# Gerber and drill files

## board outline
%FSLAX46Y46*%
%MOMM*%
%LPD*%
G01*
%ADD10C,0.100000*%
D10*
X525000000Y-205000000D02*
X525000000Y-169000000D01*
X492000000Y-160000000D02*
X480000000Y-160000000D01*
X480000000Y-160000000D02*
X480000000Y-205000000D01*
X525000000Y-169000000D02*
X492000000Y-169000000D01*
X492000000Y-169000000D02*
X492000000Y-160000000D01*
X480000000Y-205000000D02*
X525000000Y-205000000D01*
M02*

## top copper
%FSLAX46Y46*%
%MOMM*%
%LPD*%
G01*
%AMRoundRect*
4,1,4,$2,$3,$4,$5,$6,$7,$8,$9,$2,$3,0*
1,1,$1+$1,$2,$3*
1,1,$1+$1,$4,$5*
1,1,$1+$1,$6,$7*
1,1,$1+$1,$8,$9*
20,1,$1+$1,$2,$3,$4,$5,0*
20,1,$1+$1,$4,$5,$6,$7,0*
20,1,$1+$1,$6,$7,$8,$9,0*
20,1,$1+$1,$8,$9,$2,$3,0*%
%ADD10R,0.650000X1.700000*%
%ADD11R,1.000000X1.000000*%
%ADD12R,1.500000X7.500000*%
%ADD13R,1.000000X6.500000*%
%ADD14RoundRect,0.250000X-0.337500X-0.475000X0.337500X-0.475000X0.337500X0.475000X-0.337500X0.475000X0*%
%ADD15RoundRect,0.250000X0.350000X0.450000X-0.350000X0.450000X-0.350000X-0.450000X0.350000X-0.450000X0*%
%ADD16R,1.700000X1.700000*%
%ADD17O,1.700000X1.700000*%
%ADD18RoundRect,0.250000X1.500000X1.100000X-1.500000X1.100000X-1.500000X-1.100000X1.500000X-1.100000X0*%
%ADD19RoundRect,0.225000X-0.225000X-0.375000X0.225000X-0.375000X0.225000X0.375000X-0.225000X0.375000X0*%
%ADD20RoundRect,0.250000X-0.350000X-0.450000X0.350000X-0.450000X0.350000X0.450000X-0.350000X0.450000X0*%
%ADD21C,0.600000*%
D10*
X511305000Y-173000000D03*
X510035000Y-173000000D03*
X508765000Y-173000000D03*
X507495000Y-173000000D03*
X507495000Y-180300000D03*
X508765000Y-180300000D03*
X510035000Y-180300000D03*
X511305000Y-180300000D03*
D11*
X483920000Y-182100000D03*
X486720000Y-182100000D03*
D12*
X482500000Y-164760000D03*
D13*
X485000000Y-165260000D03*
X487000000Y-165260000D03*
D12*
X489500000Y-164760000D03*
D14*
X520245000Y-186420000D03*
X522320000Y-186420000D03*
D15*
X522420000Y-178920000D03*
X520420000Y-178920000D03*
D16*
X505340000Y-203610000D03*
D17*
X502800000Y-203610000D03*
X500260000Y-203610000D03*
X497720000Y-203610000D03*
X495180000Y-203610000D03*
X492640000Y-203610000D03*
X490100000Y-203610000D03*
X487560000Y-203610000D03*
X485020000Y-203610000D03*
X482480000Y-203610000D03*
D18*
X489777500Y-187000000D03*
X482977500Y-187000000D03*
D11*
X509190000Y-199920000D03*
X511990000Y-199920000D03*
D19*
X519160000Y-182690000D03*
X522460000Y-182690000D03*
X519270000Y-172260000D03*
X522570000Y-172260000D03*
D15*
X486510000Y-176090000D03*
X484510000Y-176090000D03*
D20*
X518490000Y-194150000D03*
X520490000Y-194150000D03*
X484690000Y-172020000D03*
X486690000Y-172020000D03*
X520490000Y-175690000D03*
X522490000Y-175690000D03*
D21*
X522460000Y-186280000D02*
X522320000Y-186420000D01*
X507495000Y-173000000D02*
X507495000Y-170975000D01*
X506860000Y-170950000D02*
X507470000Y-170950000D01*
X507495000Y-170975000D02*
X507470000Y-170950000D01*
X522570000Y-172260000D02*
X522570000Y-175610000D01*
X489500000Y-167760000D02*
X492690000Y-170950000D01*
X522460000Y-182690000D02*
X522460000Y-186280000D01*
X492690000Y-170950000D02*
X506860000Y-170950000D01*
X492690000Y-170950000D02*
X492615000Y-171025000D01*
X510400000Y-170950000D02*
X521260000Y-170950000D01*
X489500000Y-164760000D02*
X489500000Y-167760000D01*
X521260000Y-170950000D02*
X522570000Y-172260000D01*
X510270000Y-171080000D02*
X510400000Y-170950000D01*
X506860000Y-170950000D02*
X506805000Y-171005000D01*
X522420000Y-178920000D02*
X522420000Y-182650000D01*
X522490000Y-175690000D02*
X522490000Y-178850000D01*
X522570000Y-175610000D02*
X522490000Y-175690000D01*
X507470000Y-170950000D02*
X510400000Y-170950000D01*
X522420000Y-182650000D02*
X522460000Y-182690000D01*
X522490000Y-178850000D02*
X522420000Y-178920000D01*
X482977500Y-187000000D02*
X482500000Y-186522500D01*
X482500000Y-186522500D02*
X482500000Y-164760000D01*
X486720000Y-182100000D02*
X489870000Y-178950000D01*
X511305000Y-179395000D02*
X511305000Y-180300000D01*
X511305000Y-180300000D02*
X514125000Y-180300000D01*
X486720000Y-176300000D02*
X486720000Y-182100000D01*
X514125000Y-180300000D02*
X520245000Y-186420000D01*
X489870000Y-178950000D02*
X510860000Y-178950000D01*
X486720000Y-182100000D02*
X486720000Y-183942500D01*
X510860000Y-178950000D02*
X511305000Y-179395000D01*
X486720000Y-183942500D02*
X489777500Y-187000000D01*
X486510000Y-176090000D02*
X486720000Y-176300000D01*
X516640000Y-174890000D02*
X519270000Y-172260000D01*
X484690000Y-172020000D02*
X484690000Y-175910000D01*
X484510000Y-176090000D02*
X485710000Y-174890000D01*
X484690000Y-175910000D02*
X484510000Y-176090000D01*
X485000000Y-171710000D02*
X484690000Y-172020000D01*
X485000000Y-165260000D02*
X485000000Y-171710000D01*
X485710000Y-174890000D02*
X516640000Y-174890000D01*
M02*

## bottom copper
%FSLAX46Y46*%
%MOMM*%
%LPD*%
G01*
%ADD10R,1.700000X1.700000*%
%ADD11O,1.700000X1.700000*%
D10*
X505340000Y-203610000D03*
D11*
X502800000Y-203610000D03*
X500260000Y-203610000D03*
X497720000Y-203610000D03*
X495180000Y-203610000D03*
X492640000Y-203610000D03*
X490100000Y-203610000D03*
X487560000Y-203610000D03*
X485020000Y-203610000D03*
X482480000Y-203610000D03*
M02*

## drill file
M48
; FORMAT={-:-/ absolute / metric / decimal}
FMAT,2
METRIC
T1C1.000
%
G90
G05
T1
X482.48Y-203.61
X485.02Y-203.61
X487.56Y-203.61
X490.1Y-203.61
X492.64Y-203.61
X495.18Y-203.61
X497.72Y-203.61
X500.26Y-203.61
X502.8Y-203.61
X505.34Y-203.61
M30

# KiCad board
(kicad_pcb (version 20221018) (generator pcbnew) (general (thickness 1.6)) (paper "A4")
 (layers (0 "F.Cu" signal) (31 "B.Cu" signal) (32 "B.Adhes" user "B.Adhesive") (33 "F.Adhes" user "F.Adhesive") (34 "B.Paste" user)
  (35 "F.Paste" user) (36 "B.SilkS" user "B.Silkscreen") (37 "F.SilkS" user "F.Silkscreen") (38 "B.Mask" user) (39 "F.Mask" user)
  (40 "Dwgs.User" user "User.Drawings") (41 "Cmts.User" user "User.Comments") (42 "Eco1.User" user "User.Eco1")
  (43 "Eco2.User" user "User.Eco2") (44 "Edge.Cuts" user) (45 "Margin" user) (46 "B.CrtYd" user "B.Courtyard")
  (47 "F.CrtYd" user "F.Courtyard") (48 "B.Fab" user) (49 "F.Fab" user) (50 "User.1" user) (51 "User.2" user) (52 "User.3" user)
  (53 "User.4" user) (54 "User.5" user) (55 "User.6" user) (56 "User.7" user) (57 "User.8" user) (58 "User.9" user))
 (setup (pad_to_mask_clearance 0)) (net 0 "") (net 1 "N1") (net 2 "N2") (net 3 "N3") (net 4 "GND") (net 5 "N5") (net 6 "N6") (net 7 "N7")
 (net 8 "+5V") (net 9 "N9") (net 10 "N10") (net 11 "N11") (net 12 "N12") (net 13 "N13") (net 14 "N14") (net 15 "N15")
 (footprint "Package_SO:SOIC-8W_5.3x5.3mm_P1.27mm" (layer "F.Cu") (at 509.4 176.65 -90)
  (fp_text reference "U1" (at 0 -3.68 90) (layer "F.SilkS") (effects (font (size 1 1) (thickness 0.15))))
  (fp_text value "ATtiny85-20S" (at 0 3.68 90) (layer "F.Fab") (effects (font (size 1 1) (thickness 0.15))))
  (pad "1" smd rect (at -3.65 -1.905 270) (size 1.7 0.65) (layers "F.Cu" "F.Paste" "F.Mask") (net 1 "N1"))
  (pad "2" smd rect (at -3.65 -0.635 270) (size 1.7 0.65) (layers "F.Cu" "F.Paste" "F.Mask") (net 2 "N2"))
  (pad "3" smd rect (at -3.65 0.635 270) (size 1.7 0.65) (layers "F.Cu" "F.Paste" "F.Mask") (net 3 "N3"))
  (pad "4" smd rect (at -3.65 1.905 270) (size 1.7 0.65) (layers "F.Cu" "F.Paste" "F.Mask") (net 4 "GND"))
  (pad "5" smd rect (at 3.65 1.905 270) (size 1.7 0.65) (layers "F.Cu" "F.Paste" "F.Mask") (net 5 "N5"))
  (pad "6" smd rect (at 3.65 0.635 270) (size 1.7 0.65) (layers "F.Cu" "F.Paste" "F.Mask") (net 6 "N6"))
  (pad "7" smd rect (at 3.65 -0.635 270) (size 1.7 0.65) (layers "F.Cu" "F.Paste" "F.Mask") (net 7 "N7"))
  (pad "8" smd rect (at 3.65 -1.905 270) (size 1.7 0.65) (layers "F.Cu" "F.Paste" "F.Mask") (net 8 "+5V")))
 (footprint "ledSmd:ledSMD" (layer "F.Cu") (at 485.72 182.1)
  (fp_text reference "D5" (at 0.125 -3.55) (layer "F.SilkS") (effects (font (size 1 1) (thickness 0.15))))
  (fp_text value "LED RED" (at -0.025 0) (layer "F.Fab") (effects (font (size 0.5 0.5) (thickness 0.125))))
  (pad "1" smd rect (at -1.8 0) (size 1 1) (layers "F.Cu" "F.Paste" "F.Mask") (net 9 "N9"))
  (pad "2" smd rect (at 1 0) (size 1 1) (layers "F.Cu" "F.Paste" "F.Mask") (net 8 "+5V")))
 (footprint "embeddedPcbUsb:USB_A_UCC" (layer "F.Cu") (at 486 164.96 -90)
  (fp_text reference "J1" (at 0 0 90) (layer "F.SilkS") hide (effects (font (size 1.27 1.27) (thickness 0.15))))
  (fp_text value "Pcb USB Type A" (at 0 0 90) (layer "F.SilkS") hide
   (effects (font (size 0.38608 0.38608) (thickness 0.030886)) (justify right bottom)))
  (pad "1" smd rect (at -0.2 3.5 270) (size 7.5 1.5) (layers "F.Cu" "F.Paste" "F.Mask") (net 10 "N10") (solder_mask_margin 0.1016))
  (pad "2" smd rect (at 0.3 1 270) (size 6.5 1) (layers "F.Cu" "F.Paste" "F.Mask") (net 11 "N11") (solder_mask_margin 0.1016))
  (pad "3" smd rect (at 0.3 -1 270) (size 6.5 1) (layers "F.Cu" "F.Paste" "F.Mask") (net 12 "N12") (solder_mask_margin 0.1016))
  (pad "4" smd rect (at -0.2 -3.5 270) (size 7.5 1.5) (layers "F.Cu" "F.Paste" "F.Mask") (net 4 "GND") (solder_mask_margin 0.1016)))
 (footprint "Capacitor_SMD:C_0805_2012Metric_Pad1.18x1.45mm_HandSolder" (layer "F.Cu") (at 521.2825 186.42)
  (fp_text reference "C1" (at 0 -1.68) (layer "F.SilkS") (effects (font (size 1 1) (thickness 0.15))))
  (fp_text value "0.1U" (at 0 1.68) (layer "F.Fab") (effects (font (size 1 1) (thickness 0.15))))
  (pad "1" smd roundrect (at -1.0375 0) (size 1.175 1.45) (layers "F.Cu" "F.Paste" "F.Mask") (roundrect_rratio 0.212766) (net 8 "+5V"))
  (pad "2" smd roundrect (at 1.0375 0) (size 1.175 1.45) (layers "F.Cu" "F.Paste" "F.Mask") (roundrect_rratio 0.212766) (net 4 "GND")))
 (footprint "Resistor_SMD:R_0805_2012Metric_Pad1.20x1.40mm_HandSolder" (layer "F.Cu") (at 521.42 178.92 180)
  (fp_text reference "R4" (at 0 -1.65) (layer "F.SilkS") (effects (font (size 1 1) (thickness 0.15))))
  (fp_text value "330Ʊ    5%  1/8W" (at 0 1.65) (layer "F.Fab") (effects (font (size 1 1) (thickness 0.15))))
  (pad "1" smd roundrect (at -1 0 180) (size 1.2 1.4) (layers "F.Cu" "F.Paste" "F.Mask") (roundrect_rratio 0.208333) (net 4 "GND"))
  (pad "2" smd roundrect (at 1 0 180) (size 1.2 1.4) (layers "F.Cu" "F.Paste" "F.Mask") (roundrect_rratio 0.208333) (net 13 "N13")))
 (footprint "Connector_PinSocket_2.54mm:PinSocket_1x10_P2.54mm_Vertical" (layer "F.Cu") (at 505.34 203.61 -90)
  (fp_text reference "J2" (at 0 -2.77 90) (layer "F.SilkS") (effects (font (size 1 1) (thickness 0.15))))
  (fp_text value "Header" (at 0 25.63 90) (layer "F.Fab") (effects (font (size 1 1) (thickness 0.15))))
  (pad "1" thru_hole rect (at 0 0 270) (size 1.7 1.7) (drill 1) (layers "*.Cu" "*.Mask") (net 8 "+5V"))
  (pad "2" thru_hole oval (at 0 2.54 270) (size 1.7 1.7) (drill 1) (layers "*.Cu" "*.Mask") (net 4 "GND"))
  (pad "3" thru_hole oval (at 0 5.08 270) (size 1.7 1.7) (drill 1) (layers "*.Cu" "*.Mask") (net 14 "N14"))
  (pad "4" thru_hole oval (at 0 7.62 270) (size 1.7 1.7) (drill 1) (layers "*.Cu" "*.Mask") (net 5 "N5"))
  (pad "5" thru_hole oval (at 0 10.16 270) (size 1.7 1.7) (drill 1) (layers "*.Cu" "*.Mask") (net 6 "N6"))
  (pad "6" thru_hole oval (at 0 12.7 270) (size 1.7 1.7) (drill 1) (layers "*.Cu" "*.Mask") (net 7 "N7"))
  (pad "7" thru_hole oval (at 0 15.24 270) (size 1.7 1.7) (drill 1) (layers "*.Cu" "*.Mask") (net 2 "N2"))
  (pad "8" thru_hole oval (at 0 17.78 270) (size 1.7 1.7) (drill 1) (layers "*.Cu" "*.Mask") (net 3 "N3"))
  (pad "9" thru_hole oval (at 0 20.32 270) (size 1.7 1.7) (drill 1) (layers "*.Cu" "*.Mask") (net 1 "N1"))
  (pad "10" thru_hole oval (at 0 22.86 270) (size 1.7 1.7) (drill 1) (layers "*.Cu" "*.Mask") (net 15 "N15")))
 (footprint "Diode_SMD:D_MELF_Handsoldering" (layer "F.Cu") (at 486.3775 187 180)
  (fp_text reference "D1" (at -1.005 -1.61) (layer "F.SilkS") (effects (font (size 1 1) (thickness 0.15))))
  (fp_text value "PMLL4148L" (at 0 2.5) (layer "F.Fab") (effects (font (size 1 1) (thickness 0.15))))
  (pad "1" smd roundrect (at -3.4 0 180) (size 3.5 2.7) (layers "F.Cu" "F.Paste" "F.Mask") (roundrect_rratio 0.0925925926) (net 8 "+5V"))
  (pad "2" smd roundrect (at 3.4 0 180) (size 3.5 2.7) (layers "F.Cu" "F.Paste" "F.Mask") (roundrect_rratio 0.0925925926) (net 10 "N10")))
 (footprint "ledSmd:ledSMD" (layer "F.Cu") (at 510.99 199.92)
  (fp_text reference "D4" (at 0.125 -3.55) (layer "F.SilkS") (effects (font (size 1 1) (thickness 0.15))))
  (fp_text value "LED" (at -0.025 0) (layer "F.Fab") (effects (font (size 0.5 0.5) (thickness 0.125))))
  (pad "1" smd rect (at -1.8 0) (size 1 1) (layers "F.Cu" "F.Paste" "F.Mask") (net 13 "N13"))
  (pad "2" smd rect (at 1 0) (size 1 1) (layers "F.Cu" "F.Paste" "F.Mask") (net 6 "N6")))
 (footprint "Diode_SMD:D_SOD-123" (layer "F.Cu") (at 520.81 182.69)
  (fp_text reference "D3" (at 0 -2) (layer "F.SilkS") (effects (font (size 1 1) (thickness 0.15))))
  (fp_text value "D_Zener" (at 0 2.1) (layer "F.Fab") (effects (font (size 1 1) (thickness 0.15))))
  (pad "1" smd roundrect (at -1.65 0) (size 0.9 1.2) (layers "F.Cu" "F.Paste" "F.Mask") (roundrect_rratio 0.25) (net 12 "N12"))
  (pad "2" smd roundrect (at 1.65 0) (size 0.9 1.2) (layers "F.Cu" "F.Paste" "F.Mask") (roundrect_rratio 0.25) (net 4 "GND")))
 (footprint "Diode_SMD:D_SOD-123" (layer "F.Cu") (at 520.92 172.26)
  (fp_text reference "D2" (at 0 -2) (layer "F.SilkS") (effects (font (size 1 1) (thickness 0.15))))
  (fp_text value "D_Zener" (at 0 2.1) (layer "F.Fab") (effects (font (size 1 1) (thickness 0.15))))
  (pad "1" smd roundrect (at -1.65 0) (size 0.9 1.2) (layers "F.Cu" "F.Paste" "F.Mask") (roundrect_rratio 0.25) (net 11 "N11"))
  (pad "2" smd roundrect (at 1.65 0) (size 0.9 1.2) (layers "F.Cu" "F.Paste" "F.Mask") (roundrect_rratio 0.25) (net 4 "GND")))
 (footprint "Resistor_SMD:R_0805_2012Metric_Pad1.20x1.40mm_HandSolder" (layer "F.Cu") (at 485.51 176.09 180)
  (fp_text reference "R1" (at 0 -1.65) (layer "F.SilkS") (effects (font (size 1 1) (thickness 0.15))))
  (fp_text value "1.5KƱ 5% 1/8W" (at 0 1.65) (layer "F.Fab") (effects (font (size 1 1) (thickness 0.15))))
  (pad "1" smd roundrect (at -1 0 180) (size 1.2 1.4) (layers "F.Cu" "F.Paste" "F.Mask") (roundrect_rratio 0.208333) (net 8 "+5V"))
  (pad "2" smd roundrect (at 1 0 180) (size 1.2 1.4) (layers "F.Cu" "F.Paste" "F.Mask") (roundrect_rratio 0.208333) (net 11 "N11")))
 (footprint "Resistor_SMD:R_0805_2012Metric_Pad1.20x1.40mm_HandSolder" (layer "F.Cu") (at 519.49 194.15)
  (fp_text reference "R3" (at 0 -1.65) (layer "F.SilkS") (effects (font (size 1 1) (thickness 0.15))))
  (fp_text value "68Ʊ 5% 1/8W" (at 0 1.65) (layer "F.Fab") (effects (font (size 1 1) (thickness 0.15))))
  (pad "1" smd roundrect (at -1 0) (size 1.2 1.4) (layers "F.Cu" "F.Paste" "F.Mask") (roundrect_rratio 0.208333) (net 12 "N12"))
  (pad "2" smd roundrect (at 1 0) (size 1.2 1.4) (layers "F.Cu" "F.Paste" "F.Mask") (roundrect_rratio 0.208333) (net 3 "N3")))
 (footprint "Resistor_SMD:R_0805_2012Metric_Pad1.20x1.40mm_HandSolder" (layer "F.Cu") (at 485.69 172.02)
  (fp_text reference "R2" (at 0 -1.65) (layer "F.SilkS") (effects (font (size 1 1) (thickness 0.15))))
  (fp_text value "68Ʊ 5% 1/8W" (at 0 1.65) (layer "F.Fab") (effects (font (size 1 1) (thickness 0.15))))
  (pad "1" smd roundrect (at -1 0) (size 1.2 1.4) (layers "F.Cu" "F.Paste" "F.Mask") (roundrect_rratio 0.208333) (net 11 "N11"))
  (pad "2" smd roundrect (at 1 0) (size 1.2 1.4) (layers "F.Cu" "F.Paste" "F.Mask") (roundrect_rratio 0.208333) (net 2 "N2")))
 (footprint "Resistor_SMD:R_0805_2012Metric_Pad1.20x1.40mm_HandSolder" (layer "F.Cu") (at 521.49 175.69)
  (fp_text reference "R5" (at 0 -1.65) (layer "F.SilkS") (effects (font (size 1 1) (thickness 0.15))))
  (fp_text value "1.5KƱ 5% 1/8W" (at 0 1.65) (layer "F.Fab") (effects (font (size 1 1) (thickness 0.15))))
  (pad "1" smd roundrect (at -1 0) (size 1.2 1.4) (layers "F.Cu" "F.Paste" "F.Mask") (roundrect_rratio 0.208333) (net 9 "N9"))
  (pad "2" smd roundrect (at 1 0) (size 1.2 1.4) (layers "F.Cu" "F.Paste" "F.Mask") (roundrect_rratio 0.208333) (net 4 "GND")))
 (gr_line (start 525 205) (end 525 169) (stroke (width 0.1) (type default)) (layer "Edge.Cuts"))
 (gr_line (start 492 160) (end 480 160) (stroke (width 0.1) (type default)) (layer "Edge.Cuts"))
 (gr_line (start 480 160) (end 480 205) (stroke (width 0.1) (type default)) (layer "Edge.Cuts"))
 (gr_line (start 525 169) (end 492 169) (stroke (width 0.1) (type default)) (layer "Edge.Cuts"))
 (gr_line (start 492 169) (end 492 160) (stroke (width 0.1) (type default)) (layer "Edge.Cuts"))
 (gr_line (start 480 205) (end 525 205) (stroke (width 0.1) (type default)) (layer "Edge.Cuts"))
 (segment (start 522.46 186.28) (end 522.32 186.42) (width 0.6) (layer "F.Cu") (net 4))
 (segment (start 507.495 173) (end 507.495 170.975) (width 0.6) (layer "F.Cu") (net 4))
 (segment (start 506.86 170.95) (end 507.47 170.95) (width 0.6) (layer "F.Cu") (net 4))
 (segment (start 507.495 170.975) (end 507.47 170.95) (width 0.6) (layer "F.Cu") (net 4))
 (segment (start 522.57 172.26) (end 522.57 175.61) (width 0.6) (layer "F.Cu") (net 4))
 (segment (start 489.5 167.76) (end 492.69 170.95) (width 0.6) (layer "F.Cu") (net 4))
 (segment (start 522.46 182.69) (end 522.46 186.28) (width 0.6) (layer "F.Cu") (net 4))
 (segment (start 492.69 170.95) (end 506.86 170.95) (width 0.6) (layer "F.Cu") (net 4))
 (segment (start 492.69 170.95) (end 492.615 171.025) (width 0.6) (layer "F.Cu") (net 4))
 (segment (start 510.4 170.95) (end 521.26 170.95) (width 0.6) (layer "F.Cu") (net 4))
 (segment (start 489.5 164.76) (end 489.5 167.76) (width 0.6) (layer "F.Cu") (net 4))
 (segment (start 521.26 170.95) (end 522.57 172.26) (width 0.6) (layer "F.Cu") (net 4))
 (segment (start 510.27 171.08) (end 510.4 170.95) (width 0.6) (layer "F.Cu") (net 4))
 (segment (start 506.86 170.95) (end 506.805 171.005) (width 0.6) (layer "F.Cu") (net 4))
 (segment (start 522.42 178.92) (end 522.42 182.65) (width 0.6) (layer "F.Cu") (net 4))
 (segment (start 522.49 175.69) (end 522.49 178.85) (width 0.6) (layer "F.Cu") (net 4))
 (segment (start 522.57 175.61) (end 522.49 175.69) (width 0.6) (layer "F.Cu") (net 4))
 (segment (start 507.47 170.95) (end 510.4 170.95) (width 0.6) (layer "F.Cu") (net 4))
 (segment (start 522.42 182.65) (end 522.46 182.69) (width 0.6) (layer "F.Cu") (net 4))
 (segment (start 522.49 178.85) (end 522.42 178.92) (width 0.6) (layer "F.Cu") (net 4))
 (segment (start 482.9775 187) (end 482.5 186.5225) (width 0.6) (layer "F.Cu") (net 10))
 (segment (start 482.5 186.5225) (end 482.5 164.76) (width 0.6) (layer "F.Cu") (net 10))
 (segment (start 486.72 182.1) (end 489.87 178.95) (width 0.6) (layer "F.Cu") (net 8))
 (segment (start 511.305 179.395) (end 511.305 180.3) (width 0.6) (layer "F.Cu") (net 8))
 (segment (start 511.305 180.3) (end 514.125 180.3) (width 0.6) (layer "F.Cu") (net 8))
 (segment (start 486.72 176.3) (end 486.72 182.1) (width 0.6) (layer "F.Cu") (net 8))
 (segment (start 514.125 180.3) (end 520.245 186.42) (width 0.6) (layer "F.Cu") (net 8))
 (segment (start 489.87 178.95) (end 510.86 178.95) (width 0.6) (layer "F.Cu") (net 8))
 (segment (start 486.72 182.1) (end 486.72 183.9425) (width 0.6) (layer "F.Cu") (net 8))
 (segment (start 510.86 178.95) (end 511.305 179.395) (width 0.6) (layer "F.Cu") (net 8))
 (segment (start 486.72 183.9425) (end 489.7775 187) (width 0.6) (layer "F.Cu") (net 8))
 (segment (start 486.51 176.09) (end 486.72 176.3) (width 0.6) (layer "F.Cu") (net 8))
 (segment (start 516.64 174.89) (end 519.27 172.26) (width 0.6) (layer "F.Cu") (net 11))
 (segment (start 484.69 172.02) (end 484.69 175.91) (width 0.6) (layer "F.Cu") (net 11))
 (segment (start 484.51 176.09) (end 485.71 174.89) (width 0.6) (layer "F.Cu") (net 11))
 (segment (start 484.69 175.91) (end 484.51 176.09) (width 0.6) (layer "F.Cu") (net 11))
 (segment (start 485 171.71) (end 484.69 172.02) (width 0.6) (layer "F.Cu") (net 11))
 (segment (start 485 165.26) (end 485 171.71) (width 0.6) (layer "F.Cu") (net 11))
 (segment (start 485.71 174.89) (end 516.64 174.89) (width 0.6) (layer "F.Cu") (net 11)))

